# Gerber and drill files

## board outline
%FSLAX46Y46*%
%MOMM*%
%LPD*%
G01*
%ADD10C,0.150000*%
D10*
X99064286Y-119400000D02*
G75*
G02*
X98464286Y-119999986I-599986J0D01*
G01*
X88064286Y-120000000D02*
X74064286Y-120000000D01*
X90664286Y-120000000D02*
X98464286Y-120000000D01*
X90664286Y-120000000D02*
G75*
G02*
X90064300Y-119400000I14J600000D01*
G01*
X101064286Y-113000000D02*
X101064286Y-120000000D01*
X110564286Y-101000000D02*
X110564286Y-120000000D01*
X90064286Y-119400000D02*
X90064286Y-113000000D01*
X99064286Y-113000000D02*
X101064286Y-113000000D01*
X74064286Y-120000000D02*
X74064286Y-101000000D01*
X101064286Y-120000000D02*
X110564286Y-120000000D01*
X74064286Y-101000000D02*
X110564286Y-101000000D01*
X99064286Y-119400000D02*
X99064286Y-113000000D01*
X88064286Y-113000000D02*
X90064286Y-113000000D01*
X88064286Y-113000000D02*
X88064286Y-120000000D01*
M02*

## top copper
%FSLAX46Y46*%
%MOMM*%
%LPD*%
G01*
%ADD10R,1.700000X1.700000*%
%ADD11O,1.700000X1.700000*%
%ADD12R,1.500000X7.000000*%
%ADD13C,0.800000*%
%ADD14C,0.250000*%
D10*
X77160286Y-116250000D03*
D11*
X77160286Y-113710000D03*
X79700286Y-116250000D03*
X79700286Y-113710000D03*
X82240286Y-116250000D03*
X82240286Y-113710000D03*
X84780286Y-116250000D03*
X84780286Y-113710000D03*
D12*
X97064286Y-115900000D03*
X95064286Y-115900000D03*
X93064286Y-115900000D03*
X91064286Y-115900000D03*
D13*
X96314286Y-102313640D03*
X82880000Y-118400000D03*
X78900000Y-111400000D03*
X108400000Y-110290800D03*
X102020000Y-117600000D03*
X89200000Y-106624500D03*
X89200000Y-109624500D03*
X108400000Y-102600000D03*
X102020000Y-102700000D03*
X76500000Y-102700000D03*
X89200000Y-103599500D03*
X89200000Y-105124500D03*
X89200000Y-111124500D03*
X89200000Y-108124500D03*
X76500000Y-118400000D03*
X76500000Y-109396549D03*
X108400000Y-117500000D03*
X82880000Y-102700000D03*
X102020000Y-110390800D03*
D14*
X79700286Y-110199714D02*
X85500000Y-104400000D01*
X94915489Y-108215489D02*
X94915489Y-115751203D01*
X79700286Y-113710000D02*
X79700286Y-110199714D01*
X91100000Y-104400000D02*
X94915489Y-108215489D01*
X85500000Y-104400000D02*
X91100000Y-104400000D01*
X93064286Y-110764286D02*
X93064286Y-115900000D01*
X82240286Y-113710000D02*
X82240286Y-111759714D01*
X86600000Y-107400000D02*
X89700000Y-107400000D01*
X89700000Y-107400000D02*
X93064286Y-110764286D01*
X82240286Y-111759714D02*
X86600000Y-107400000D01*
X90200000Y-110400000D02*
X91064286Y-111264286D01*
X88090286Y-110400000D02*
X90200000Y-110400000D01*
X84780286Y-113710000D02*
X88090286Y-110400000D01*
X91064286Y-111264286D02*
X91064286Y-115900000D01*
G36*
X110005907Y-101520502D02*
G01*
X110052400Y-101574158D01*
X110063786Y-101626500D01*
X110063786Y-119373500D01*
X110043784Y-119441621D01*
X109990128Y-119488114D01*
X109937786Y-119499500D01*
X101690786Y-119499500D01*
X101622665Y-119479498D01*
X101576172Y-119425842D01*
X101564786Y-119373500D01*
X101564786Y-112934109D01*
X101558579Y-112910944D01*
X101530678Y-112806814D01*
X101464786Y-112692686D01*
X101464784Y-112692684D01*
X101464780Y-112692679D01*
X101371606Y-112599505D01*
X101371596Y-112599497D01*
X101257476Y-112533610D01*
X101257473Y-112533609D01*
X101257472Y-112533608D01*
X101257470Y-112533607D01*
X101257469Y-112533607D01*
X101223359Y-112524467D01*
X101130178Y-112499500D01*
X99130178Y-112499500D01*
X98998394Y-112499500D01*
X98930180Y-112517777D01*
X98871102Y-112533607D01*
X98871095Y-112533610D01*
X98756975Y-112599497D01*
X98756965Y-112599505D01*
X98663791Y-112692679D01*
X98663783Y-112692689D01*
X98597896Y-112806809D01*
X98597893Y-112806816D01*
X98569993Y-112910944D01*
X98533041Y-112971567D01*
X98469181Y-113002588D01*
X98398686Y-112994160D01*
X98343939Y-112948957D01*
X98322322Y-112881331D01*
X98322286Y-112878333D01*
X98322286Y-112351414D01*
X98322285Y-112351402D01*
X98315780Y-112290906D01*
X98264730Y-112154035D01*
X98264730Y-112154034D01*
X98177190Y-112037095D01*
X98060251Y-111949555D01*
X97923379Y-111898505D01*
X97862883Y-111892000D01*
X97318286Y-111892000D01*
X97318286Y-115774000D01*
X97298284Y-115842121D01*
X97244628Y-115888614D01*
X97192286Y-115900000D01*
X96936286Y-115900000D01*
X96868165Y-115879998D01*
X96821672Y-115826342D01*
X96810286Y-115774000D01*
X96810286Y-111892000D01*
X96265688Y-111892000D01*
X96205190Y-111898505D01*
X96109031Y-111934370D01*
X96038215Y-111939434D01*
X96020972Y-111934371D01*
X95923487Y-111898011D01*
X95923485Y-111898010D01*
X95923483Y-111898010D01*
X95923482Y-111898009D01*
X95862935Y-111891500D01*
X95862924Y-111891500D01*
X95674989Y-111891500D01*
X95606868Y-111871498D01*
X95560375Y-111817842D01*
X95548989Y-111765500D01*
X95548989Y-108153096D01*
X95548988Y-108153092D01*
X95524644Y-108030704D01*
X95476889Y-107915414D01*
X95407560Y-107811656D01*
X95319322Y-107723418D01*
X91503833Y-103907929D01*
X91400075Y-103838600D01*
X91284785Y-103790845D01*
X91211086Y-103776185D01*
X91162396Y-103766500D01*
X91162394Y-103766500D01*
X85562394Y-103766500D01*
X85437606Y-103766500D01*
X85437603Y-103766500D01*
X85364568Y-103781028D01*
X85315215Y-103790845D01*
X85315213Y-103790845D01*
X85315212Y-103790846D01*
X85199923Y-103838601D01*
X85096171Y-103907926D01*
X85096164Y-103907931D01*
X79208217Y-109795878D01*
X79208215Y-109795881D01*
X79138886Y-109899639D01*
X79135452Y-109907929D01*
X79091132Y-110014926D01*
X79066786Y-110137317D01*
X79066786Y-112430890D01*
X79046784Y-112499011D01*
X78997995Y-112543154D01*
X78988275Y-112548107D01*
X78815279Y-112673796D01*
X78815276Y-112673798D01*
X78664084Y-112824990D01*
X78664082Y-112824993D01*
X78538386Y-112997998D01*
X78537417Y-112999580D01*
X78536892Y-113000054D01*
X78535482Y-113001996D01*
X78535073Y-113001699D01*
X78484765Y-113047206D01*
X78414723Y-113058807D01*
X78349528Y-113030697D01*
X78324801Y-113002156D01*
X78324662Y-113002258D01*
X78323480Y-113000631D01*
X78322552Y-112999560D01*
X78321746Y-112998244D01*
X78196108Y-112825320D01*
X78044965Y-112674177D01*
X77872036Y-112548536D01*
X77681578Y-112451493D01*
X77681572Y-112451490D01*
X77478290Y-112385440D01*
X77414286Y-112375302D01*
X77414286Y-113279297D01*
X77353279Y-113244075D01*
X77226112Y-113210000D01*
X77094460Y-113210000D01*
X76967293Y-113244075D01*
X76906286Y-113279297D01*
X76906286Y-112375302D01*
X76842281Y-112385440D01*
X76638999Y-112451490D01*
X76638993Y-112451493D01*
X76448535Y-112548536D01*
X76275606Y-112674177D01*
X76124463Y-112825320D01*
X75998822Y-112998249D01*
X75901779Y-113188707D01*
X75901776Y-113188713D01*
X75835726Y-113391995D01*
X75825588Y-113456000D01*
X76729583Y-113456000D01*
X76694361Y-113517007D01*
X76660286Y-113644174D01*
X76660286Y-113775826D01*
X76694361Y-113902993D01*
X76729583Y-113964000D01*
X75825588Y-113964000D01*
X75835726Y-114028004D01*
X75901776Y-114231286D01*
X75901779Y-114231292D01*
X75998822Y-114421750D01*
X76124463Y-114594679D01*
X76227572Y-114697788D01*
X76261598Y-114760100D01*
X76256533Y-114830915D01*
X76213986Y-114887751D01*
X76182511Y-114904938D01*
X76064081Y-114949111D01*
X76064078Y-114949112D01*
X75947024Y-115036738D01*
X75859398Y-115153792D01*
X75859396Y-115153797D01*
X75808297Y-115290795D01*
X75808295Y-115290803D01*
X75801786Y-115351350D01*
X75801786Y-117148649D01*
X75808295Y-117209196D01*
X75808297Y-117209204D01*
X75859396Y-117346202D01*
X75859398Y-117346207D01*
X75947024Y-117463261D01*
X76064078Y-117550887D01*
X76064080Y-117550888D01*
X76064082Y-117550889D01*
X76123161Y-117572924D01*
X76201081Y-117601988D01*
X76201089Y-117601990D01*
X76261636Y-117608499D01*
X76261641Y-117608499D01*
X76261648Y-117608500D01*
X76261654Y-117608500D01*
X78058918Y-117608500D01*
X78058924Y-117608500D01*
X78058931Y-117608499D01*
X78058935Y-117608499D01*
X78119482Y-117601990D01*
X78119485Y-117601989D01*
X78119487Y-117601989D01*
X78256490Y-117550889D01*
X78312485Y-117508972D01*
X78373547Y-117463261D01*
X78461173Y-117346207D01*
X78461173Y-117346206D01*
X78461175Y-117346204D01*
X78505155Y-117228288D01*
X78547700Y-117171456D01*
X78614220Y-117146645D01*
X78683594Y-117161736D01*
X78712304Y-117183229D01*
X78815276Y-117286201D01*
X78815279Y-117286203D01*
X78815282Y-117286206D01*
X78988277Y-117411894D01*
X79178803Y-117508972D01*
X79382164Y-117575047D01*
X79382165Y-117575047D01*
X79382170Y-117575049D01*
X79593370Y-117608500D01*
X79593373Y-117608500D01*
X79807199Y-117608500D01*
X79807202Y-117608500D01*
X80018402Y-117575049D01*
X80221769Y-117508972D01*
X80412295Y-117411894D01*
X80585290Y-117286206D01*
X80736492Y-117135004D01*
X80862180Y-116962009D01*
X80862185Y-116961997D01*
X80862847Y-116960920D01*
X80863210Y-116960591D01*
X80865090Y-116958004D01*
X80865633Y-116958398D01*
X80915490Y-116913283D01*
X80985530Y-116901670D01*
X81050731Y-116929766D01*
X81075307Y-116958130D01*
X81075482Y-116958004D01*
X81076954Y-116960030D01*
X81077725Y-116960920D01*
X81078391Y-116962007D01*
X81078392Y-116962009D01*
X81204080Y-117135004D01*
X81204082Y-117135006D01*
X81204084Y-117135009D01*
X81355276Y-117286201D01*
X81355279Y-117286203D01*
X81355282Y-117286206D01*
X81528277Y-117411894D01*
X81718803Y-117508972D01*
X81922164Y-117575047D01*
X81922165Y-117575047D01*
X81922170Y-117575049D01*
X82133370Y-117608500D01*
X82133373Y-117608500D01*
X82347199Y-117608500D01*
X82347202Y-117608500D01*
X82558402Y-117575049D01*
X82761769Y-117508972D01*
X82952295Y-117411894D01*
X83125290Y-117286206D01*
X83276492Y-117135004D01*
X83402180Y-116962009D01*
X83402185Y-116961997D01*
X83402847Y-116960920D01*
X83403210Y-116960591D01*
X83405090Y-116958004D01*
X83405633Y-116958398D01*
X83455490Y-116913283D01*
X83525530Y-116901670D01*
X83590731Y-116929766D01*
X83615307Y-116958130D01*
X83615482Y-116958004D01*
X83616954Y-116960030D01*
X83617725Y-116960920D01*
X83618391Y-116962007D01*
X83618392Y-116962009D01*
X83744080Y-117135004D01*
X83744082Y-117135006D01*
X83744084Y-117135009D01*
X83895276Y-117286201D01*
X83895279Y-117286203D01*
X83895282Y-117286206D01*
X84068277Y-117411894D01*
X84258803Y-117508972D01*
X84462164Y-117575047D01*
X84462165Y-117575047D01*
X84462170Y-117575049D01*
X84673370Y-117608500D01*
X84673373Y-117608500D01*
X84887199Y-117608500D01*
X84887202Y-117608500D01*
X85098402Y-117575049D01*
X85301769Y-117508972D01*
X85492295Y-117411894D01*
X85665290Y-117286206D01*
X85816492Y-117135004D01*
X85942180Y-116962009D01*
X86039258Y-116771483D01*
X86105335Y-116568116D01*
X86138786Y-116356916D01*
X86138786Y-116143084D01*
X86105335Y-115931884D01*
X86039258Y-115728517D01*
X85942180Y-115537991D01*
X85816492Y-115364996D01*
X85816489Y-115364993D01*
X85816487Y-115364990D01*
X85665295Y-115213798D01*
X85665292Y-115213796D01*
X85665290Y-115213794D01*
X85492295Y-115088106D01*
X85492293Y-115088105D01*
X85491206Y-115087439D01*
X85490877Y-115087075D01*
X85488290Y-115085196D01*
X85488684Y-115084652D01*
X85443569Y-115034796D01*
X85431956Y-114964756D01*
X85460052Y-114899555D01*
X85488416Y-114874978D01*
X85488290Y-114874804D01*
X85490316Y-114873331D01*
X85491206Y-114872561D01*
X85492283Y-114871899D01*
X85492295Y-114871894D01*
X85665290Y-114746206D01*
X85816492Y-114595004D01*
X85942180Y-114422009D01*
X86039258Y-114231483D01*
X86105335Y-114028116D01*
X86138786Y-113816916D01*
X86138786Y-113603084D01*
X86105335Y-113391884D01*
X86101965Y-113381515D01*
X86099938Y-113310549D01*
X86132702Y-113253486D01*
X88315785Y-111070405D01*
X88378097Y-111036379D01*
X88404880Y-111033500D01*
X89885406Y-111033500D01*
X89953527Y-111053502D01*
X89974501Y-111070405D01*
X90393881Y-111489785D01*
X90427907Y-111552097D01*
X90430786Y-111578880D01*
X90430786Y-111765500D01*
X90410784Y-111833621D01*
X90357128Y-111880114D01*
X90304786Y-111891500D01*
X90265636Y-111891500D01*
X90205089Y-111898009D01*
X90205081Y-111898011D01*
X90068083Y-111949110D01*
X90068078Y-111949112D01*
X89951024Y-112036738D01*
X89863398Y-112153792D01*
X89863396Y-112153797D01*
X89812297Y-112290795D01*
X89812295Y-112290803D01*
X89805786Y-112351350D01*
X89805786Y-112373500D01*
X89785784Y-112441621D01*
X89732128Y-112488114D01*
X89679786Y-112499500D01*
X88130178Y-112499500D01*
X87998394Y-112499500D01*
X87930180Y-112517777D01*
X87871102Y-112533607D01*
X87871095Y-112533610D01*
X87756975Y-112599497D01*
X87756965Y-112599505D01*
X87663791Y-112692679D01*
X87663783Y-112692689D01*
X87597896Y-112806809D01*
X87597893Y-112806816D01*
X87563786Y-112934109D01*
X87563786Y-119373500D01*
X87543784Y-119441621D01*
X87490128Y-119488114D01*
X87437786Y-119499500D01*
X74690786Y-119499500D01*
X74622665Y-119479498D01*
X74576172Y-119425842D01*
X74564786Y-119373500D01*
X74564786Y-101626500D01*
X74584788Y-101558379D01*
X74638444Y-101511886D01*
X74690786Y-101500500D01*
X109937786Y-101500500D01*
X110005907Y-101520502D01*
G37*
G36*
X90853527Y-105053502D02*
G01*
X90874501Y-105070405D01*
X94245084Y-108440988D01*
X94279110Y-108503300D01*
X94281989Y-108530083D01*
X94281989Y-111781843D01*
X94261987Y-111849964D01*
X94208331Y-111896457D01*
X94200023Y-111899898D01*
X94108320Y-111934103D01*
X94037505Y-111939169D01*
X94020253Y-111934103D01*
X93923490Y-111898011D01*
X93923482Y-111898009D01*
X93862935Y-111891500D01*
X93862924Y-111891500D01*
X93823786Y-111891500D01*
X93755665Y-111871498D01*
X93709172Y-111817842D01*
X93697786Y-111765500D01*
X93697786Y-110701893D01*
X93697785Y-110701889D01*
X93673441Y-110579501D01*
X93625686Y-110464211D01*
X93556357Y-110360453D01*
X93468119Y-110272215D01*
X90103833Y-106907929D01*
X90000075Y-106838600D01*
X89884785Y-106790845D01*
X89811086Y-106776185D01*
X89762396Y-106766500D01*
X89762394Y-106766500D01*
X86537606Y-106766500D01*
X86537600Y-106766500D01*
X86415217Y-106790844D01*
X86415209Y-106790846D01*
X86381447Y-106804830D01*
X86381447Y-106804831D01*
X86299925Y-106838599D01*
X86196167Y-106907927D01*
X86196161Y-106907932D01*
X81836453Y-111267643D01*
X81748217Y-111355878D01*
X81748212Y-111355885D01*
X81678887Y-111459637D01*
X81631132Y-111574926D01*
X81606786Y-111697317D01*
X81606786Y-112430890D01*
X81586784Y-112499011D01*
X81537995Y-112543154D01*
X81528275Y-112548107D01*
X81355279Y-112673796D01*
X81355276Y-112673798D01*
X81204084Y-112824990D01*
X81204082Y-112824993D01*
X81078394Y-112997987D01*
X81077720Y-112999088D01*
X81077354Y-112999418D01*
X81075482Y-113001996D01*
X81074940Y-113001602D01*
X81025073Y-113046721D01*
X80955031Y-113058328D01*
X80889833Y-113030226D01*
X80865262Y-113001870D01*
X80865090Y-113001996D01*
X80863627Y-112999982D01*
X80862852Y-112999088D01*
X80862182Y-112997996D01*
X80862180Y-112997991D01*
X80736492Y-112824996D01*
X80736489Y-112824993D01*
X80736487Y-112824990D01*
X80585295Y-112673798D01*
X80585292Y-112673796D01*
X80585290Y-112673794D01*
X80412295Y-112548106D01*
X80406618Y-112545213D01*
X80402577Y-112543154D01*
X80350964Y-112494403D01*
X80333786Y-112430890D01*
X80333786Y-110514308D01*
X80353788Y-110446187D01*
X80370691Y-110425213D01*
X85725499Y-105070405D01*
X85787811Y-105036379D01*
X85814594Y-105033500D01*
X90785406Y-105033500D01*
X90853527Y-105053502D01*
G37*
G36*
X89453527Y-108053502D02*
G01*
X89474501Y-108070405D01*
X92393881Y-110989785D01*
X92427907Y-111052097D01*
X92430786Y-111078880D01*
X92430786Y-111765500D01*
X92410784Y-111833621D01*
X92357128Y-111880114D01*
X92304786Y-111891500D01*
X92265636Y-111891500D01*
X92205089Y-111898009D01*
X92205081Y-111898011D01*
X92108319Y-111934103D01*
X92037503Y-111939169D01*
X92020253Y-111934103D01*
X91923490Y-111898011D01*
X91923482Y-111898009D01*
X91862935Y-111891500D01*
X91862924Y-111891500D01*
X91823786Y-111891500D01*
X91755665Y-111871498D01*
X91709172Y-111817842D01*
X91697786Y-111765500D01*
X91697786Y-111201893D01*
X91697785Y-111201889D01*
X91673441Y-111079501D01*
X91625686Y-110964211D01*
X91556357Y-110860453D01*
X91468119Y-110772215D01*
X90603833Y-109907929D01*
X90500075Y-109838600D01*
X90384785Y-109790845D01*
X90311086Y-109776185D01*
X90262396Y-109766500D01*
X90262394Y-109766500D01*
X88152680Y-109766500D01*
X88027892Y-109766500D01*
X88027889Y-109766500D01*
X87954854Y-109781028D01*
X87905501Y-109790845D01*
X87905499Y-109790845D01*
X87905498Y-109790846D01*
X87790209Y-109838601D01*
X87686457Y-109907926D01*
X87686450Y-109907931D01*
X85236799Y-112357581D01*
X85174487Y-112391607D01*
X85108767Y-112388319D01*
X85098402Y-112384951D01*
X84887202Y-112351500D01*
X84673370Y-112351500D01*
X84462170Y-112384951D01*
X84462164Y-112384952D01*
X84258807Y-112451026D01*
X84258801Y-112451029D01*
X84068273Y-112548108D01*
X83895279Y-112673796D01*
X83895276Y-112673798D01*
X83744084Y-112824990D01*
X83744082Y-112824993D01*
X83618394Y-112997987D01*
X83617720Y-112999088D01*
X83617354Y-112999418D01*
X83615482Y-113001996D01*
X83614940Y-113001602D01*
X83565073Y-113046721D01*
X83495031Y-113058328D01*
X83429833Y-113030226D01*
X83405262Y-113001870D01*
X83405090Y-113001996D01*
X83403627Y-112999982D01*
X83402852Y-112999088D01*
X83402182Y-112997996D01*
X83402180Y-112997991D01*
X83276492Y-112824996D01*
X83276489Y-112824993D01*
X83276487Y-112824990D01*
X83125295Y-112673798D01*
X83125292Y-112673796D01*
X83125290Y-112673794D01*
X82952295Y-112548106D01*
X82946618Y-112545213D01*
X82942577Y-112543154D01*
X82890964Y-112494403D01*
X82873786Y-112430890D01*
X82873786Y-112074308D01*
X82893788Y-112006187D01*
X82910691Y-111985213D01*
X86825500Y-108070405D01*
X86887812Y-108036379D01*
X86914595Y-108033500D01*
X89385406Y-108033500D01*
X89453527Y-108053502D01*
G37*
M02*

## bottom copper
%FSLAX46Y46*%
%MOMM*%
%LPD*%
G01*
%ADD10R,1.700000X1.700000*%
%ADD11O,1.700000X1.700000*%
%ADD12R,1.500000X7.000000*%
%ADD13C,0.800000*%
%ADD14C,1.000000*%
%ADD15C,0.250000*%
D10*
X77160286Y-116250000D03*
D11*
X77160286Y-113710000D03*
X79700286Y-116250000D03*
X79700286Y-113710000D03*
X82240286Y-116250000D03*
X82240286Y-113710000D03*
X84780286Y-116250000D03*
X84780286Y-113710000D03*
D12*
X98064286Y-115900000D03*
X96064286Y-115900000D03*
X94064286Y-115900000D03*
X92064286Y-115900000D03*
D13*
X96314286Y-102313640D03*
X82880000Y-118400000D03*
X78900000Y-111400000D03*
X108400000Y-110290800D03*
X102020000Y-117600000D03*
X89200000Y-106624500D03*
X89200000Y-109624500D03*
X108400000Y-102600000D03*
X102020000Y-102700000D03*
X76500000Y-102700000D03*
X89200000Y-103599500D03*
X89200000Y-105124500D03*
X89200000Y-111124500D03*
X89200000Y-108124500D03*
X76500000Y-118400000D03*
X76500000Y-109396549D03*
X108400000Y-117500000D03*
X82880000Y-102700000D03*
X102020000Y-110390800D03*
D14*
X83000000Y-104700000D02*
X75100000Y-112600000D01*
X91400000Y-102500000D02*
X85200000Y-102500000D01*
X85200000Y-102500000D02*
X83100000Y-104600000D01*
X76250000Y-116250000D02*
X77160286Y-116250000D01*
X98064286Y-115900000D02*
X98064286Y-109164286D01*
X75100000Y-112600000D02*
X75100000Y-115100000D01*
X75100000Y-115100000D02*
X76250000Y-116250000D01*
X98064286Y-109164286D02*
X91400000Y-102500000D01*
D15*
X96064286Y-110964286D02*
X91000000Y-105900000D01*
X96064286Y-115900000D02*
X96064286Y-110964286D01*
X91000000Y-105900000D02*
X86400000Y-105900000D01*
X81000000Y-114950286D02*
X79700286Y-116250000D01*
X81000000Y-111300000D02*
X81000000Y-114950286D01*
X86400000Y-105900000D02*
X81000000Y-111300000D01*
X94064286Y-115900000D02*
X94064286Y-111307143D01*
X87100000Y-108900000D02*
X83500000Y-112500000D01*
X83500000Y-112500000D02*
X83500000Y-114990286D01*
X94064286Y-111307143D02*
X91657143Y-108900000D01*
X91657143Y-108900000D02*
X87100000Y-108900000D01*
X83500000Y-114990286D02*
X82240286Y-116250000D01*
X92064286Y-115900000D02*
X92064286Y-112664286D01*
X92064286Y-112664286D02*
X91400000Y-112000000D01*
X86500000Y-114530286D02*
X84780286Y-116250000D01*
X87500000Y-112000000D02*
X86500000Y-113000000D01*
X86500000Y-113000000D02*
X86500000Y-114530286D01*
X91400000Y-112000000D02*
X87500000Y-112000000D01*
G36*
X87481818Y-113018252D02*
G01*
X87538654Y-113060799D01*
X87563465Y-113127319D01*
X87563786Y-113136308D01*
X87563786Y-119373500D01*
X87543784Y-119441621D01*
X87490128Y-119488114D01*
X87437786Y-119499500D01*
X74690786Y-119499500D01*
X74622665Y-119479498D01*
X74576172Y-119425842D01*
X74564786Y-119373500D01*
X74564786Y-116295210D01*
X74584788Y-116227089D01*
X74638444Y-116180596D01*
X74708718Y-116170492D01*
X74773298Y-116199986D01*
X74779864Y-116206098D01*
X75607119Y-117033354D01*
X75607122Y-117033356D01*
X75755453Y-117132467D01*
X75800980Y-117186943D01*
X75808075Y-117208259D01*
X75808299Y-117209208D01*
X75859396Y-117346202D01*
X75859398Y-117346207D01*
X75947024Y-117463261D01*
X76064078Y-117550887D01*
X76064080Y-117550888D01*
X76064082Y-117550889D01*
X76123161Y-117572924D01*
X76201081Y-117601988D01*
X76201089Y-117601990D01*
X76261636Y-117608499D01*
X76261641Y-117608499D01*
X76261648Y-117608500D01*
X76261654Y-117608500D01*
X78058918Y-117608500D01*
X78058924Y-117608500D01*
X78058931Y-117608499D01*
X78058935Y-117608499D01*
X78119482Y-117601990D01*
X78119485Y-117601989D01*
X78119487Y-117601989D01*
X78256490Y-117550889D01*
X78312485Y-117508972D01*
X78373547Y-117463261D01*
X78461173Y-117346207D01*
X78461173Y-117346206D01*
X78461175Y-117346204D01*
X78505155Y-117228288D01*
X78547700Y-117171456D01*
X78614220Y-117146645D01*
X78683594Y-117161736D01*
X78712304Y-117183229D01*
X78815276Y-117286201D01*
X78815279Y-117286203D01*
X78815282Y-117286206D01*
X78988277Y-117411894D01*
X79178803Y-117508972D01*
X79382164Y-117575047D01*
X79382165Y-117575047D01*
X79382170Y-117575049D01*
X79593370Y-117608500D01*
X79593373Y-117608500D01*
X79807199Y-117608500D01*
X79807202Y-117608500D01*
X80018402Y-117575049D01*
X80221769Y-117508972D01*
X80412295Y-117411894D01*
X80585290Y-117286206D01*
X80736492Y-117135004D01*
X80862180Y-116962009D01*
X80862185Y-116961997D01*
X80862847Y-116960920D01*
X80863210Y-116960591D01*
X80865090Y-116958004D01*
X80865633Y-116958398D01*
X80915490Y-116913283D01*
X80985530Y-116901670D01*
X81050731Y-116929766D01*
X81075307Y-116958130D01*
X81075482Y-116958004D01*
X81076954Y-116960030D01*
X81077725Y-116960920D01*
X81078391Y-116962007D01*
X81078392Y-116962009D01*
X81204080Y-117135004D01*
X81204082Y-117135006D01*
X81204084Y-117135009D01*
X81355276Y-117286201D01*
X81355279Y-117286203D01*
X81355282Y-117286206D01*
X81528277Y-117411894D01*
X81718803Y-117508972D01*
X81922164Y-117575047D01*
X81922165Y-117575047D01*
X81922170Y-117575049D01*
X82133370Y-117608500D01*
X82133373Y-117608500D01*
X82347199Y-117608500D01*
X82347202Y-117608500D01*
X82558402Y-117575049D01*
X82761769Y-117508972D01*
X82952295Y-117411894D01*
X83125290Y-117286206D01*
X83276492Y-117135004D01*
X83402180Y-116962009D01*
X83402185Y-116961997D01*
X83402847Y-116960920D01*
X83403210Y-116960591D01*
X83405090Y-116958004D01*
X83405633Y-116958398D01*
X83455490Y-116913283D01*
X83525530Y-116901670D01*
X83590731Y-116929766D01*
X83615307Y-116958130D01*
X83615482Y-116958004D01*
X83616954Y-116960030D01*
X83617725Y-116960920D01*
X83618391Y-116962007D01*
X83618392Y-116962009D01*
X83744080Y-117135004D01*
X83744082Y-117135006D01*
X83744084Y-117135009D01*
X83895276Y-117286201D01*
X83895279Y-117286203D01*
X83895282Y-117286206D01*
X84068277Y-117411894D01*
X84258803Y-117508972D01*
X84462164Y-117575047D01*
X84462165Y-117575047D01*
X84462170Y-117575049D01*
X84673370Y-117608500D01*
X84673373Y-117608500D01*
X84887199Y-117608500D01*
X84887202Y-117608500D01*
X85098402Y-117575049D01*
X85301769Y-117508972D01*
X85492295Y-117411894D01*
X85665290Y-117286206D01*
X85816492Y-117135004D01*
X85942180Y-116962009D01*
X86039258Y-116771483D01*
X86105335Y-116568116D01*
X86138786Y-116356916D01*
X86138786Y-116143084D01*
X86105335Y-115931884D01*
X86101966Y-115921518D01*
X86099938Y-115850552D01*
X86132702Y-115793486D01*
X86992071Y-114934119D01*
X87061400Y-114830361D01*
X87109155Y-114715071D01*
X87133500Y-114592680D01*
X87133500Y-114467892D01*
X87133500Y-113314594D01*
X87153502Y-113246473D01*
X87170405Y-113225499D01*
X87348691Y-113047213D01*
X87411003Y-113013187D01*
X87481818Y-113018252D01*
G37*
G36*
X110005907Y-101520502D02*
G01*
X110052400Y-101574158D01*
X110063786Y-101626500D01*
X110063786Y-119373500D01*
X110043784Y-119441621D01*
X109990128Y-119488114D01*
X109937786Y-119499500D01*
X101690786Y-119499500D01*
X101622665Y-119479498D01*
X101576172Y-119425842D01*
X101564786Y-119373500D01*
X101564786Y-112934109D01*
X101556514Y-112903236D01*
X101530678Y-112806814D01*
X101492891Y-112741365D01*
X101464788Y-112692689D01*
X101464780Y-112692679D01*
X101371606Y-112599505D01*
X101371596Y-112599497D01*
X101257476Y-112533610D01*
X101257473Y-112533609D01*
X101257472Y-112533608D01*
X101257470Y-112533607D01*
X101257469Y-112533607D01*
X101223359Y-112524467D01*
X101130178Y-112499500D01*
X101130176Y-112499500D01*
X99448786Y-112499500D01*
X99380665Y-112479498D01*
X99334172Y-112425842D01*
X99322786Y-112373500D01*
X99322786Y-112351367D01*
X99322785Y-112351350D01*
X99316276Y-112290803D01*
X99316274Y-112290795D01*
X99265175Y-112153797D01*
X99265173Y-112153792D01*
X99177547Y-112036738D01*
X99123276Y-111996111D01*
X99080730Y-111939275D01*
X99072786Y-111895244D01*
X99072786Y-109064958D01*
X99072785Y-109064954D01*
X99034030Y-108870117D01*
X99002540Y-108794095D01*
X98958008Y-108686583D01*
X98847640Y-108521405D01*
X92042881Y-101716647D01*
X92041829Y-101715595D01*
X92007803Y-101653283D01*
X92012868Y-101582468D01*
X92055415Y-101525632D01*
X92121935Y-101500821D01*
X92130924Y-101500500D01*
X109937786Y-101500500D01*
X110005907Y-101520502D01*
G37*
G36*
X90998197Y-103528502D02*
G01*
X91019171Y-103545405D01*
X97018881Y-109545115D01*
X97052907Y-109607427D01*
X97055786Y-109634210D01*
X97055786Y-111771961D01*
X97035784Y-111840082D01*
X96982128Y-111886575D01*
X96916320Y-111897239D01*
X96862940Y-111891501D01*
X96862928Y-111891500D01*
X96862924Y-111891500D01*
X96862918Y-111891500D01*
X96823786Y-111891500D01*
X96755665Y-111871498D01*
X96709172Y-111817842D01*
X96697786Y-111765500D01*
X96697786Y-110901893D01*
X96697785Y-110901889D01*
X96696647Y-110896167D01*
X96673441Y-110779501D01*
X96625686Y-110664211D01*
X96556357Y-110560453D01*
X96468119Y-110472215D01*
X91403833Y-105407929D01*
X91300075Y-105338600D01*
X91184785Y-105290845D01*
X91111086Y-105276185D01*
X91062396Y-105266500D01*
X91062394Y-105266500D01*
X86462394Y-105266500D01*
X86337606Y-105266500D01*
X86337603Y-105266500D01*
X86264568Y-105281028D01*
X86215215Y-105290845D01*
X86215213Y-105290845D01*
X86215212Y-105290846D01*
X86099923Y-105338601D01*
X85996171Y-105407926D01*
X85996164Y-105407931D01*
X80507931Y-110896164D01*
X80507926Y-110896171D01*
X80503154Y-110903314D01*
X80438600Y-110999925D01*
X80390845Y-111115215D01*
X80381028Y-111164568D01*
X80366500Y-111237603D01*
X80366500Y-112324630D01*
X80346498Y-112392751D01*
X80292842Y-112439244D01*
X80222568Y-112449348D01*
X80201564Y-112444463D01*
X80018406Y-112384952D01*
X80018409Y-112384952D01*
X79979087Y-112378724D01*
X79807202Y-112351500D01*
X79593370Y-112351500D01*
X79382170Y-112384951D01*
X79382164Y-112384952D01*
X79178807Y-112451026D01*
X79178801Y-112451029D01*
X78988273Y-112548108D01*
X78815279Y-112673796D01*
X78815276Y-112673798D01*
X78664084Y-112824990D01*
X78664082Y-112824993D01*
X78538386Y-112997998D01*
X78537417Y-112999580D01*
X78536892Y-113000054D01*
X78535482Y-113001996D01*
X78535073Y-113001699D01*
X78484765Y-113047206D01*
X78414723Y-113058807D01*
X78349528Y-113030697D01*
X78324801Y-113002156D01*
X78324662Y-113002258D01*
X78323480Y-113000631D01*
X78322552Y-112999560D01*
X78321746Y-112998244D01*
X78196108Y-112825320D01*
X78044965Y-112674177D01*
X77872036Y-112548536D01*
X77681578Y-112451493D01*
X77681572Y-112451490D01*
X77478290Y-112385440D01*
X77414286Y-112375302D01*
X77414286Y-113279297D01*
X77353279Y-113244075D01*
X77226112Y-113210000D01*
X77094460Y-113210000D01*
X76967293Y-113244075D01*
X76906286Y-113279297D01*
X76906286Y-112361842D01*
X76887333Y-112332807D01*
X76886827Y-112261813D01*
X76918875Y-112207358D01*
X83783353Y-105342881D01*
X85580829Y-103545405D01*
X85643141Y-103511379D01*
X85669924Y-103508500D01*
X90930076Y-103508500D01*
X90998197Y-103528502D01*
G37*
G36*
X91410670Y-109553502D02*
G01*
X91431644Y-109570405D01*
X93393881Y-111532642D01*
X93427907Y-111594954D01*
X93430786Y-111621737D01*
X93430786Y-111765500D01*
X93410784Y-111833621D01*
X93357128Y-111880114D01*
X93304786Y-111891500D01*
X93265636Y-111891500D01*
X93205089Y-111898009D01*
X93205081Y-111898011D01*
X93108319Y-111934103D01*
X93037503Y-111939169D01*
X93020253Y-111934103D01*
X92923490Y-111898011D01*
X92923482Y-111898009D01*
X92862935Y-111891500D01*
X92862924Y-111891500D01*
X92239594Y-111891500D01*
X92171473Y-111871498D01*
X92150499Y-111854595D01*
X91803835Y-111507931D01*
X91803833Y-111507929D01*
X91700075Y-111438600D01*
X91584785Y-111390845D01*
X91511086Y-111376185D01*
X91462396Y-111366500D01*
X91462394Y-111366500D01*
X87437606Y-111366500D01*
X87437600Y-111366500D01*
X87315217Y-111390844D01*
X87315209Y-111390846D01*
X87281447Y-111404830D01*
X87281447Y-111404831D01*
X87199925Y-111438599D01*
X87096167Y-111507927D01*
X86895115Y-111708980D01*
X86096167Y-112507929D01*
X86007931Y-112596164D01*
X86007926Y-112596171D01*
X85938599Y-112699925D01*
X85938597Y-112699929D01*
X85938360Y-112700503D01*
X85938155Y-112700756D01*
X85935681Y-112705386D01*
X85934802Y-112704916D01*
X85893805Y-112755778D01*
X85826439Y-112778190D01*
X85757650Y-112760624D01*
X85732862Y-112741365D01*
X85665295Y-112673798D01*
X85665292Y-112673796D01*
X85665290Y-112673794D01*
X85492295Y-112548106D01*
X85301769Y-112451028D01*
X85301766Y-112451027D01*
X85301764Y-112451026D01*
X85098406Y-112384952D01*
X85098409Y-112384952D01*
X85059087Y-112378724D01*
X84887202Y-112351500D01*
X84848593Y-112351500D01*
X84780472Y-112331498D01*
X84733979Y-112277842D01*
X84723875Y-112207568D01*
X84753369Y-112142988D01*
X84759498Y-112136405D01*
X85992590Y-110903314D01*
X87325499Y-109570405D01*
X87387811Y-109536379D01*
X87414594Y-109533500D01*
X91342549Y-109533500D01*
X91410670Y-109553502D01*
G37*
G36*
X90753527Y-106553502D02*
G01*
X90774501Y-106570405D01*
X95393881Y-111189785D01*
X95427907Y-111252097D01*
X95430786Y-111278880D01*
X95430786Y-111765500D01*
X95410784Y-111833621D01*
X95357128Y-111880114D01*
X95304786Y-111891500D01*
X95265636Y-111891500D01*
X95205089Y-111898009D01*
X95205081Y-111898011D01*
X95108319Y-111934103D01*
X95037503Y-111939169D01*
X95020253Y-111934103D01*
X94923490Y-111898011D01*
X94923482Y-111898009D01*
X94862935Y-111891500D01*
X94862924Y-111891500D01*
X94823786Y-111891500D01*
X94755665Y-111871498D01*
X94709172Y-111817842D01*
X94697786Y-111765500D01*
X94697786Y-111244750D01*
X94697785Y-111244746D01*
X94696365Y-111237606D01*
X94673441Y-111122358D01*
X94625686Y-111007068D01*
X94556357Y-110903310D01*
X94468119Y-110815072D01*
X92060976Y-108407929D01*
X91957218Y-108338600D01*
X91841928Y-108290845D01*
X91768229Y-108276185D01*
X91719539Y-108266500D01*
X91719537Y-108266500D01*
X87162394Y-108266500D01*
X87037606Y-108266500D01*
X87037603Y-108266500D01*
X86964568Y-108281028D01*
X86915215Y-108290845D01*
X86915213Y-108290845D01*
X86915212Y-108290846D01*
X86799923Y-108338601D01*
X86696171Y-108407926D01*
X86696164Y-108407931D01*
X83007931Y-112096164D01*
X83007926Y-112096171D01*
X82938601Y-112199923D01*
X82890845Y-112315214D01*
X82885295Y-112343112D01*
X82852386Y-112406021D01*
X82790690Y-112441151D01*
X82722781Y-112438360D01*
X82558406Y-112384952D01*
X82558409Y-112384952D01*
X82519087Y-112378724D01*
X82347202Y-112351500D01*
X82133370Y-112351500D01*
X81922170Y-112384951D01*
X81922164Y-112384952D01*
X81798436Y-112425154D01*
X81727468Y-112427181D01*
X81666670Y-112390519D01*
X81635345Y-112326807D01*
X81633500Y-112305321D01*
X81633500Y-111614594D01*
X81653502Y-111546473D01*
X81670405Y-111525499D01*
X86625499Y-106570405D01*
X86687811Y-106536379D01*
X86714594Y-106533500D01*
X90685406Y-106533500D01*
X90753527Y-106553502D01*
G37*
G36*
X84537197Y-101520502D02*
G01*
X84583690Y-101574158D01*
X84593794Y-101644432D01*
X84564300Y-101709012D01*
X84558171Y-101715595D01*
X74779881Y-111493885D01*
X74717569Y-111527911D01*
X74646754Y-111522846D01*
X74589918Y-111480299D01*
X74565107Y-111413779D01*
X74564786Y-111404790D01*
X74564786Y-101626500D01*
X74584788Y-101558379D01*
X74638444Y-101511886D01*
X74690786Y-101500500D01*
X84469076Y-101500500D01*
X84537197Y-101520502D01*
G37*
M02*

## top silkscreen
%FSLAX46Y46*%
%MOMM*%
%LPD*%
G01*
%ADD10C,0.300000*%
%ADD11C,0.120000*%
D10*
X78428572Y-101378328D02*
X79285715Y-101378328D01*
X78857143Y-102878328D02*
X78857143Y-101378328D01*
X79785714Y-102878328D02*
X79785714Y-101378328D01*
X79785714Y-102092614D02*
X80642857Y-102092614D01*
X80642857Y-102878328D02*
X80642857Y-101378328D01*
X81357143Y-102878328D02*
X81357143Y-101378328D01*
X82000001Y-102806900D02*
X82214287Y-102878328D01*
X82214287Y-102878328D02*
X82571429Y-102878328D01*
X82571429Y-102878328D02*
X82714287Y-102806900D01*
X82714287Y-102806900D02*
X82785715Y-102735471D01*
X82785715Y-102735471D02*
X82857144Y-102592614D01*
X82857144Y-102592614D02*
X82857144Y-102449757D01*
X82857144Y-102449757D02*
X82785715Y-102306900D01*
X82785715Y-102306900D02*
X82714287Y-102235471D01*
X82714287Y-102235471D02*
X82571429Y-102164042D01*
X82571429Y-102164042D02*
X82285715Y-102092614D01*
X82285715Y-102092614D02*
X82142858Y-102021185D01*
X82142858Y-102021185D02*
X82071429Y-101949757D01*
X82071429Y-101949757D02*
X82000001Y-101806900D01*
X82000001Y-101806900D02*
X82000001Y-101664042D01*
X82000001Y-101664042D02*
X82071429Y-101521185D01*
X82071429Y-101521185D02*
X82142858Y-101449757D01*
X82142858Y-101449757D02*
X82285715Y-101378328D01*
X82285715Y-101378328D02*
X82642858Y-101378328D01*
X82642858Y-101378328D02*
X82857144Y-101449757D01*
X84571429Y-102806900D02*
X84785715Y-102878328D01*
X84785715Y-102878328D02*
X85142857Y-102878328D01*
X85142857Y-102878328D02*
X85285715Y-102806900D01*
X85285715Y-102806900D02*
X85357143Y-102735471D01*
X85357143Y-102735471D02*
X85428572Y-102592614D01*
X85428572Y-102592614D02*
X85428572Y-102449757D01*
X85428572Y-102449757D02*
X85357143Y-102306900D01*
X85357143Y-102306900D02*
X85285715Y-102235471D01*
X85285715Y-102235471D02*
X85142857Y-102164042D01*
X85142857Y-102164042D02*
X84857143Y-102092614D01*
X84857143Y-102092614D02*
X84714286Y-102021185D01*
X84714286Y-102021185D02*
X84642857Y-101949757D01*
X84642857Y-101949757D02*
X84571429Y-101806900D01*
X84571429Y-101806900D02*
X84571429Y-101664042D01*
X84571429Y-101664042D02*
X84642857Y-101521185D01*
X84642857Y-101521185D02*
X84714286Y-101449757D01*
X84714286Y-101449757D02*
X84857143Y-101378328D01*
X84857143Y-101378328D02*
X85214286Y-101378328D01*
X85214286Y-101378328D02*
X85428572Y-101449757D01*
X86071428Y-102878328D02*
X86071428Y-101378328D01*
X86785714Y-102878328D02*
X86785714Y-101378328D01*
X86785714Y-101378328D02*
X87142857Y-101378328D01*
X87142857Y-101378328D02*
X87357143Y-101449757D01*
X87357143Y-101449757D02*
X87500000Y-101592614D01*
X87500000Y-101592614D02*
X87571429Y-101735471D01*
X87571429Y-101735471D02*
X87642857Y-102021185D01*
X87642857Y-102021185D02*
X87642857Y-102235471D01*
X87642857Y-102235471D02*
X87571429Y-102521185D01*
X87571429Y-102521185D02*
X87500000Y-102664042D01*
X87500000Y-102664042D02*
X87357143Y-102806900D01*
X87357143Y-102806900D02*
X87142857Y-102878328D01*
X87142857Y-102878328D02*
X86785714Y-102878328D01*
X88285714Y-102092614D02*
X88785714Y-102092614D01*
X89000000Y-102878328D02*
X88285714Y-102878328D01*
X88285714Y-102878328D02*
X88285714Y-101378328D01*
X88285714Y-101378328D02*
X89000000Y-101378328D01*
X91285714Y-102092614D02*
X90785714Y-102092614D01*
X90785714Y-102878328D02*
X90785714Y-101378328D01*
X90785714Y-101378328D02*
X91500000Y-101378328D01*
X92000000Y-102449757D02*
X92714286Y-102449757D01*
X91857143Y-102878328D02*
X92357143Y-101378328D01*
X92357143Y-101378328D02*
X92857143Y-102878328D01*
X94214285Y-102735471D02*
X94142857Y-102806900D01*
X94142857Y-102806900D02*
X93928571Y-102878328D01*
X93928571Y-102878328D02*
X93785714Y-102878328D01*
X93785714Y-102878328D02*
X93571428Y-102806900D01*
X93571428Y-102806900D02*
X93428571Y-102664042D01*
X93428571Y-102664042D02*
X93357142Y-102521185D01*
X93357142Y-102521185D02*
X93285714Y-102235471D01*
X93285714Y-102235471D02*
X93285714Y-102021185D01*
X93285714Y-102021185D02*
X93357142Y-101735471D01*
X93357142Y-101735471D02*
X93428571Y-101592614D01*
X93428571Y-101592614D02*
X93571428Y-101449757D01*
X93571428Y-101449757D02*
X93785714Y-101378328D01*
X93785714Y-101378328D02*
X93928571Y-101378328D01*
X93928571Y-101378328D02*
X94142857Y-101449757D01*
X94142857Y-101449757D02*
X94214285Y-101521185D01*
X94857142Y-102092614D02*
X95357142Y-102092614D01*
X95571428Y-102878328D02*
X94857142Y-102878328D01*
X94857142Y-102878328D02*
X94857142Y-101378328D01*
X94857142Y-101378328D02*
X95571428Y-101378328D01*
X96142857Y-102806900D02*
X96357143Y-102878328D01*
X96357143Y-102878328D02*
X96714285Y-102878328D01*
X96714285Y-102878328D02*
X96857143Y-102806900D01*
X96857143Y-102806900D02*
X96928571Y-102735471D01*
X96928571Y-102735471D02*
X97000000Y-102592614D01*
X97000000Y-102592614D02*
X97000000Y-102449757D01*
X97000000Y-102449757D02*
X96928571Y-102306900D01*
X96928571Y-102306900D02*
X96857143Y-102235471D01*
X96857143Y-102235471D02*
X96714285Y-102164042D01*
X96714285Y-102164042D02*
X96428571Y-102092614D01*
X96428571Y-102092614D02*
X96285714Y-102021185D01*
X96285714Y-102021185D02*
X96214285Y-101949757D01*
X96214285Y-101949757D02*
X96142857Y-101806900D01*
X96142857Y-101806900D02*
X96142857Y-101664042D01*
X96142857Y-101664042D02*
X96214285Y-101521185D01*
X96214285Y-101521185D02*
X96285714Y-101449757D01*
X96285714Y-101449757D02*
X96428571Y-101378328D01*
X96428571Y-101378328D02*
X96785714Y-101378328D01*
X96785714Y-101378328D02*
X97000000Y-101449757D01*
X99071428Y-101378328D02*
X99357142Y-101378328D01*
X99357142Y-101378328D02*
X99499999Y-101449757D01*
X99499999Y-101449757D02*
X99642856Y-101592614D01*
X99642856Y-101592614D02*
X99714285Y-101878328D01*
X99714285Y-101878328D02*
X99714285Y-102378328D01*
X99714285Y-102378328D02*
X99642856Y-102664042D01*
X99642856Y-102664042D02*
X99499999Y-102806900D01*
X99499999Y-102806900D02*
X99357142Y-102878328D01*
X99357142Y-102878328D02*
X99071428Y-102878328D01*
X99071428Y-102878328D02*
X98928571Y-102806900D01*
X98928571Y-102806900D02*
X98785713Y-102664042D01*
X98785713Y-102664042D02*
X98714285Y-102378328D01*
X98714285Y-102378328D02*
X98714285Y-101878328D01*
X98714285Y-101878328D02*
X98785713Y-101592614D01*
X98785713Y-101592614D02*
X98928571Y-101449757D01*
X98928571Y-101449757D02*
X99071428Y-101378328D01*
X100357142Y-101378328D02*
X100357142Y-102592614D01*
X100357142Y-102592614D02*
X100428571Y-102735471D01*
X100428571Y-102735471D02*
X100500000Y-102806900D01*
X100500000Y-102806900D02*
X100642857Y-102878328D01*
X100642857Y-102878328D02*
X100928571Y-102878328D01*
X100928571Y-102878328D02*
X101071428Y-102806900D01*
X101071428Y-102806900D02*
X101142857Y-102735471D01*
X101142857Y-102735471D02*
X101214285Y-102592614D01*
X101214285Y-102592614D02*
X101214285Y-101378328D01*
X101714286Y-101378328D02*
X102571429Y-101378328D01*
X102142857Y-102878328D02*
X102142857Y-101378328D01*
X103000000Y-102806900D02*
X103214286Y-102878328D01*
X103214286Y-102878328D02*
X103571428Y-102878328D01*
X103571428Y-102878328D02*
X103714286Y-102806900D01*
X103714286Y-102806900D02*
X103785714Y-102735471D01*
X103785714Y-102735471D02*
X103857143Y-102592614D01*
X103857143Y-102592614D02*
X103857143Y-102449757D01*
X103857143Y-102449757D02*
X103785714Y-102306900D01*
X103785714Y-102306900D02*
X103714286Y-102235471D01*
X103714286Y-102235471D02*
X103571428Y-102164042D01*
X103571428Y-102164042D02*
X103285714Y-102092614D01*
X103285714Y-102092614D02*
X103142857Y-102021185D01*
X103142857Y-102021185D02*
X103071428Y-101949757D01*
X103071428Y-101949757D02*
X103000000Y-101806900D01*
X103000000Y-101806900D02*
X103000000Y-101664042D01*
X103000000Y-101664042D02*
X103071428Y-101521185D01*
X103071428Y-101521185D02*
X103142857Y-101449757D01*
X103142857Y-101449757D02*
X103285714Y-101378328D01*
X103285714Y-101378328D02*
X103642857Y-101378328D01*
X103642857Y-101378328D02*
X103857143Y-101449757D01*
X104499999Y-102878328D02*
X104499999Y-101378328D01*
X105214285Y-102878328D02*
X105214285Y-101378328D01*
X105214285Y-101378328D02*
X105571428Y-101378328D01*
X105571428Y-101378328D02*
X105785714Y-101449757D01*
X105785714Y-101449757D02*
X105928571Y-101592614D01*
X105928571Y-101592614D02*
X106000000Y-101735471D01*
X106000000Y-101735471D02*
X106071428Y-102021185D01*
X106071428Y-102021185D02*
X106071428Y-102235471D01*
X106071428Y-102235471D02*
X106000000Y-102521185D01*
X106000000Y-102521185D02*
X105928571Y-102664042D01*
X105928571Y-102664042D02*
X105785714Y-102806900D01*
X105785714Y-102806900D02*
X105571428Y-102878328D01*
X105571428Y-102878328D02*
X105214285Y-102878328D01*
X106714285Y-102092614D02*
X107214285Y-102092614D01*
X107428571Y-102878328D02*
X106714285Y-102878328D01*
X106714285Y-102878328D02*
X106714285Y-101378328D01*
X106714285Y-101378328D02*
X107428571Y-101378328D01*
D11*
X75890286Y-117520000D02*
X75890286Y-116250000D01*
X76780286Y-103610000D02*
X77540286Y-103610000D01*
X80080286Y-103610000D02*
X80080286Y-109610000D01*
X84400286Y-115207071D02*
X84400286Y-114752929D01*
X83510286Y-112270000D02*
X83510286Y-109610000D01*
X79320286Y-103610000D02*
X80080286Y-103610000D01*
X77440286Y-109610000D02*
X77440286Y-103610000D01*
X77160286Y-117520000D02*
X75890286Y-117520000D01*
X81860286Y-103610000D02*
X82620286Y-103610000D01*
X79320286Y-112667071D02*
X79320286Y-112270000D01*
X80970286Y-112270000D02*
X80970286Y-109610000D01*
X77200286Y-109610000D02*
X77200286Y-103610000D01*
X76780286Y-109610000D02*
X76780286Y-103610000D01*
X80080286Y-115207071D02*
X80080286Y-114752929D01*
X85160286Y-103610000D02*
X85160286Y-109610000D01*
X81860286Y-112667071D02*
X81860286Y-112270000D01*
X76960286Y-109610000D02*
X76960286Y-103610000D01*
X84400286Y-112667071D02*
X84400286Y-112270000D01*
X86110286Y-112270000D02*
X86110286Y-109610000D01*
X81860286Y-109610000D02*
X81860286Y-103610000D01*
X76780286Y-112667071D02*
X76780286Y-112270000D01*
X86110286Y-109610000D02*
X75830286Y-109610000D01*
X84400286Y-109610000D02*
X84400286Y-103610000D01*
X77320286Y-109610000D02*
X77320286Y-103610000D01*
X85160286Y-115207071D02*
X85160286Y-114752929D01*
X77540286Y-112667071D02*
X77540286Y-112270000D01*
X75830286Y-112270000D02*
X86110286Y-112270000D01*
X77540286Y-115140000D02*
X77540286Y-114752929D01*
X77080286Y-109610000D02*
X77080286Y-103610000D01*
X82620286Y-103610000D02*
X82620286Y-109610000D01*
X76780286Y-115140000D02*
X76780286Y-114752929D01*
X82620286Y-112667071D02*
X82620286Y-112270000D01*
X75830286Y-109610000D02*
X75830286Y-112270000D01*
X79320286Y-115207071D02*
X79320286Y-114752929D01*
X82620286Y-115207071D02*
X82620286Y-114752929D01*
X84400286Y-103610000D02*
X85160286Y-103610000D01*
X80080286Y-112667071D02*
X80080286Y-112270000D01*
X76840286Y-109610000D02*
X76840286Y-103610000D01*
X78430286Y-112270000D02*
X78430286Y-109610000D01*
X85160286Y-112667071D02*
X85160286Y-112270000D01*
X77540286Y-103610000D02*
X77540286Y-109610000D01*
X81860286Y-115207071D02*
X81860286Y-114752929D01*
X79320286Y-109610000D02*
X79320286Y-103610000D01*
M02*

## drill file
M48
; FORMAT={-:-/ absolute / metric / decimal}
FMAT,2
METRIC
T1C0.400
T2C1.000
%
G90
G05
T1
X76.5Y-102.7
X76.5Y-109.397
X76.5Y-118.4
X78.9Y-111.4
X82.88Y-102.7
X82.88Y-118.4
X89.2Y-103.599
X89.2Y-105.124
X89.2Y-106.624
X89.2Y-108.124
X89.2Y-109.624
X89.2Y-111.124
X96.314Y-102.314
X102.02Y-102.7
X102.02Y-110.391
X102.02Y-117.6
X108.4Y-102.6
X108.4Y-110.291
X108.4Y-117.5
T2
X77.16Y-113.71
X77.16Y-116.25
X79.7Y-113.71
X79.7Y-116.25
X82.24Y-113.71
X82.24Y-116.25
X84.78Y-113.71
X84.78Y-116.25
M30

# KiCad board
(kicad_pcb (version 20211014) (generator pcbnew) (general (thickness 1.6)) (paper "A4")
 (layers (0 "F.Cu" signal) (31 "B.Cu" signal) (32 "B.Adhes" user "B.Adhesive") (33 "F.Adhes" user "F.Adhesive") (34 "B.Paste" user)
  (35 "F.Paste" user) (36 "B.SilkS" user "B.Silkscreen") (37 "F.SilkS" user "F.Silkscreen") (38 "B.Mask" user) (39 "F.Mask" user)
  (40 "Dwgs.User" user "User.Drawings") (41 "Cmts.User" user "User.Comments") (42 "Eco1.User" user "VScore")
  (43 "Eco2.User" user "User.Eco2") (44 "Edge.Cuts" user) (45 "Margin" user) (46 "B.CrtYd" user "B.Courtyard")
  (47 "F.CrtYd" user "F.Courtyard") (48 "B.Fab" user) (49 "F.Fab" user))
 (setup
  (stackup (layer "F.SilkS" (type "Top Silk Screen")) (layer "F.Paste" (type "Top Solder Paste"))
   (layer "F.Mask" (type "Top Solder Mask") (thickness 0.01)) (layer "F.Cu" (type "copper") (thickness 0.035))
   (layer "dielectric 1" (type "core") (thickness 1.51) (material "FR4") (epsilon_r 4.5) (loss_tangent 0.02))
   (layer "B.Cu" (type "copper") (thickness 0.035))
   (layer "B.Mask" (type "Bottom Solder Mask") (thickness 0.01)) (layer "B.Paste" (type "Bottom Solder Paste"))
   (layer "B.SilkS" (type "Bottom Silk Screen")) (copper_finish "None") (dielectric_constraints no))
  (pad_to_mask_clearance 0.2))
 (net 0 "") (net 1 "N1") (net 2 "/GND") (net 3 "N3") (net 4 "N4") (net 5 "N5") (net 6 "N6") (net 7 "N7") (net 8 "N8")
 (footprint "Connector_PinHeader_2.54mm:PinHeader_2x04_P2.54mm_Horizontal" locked (layer "F.Cu") (at 77.160286 116.25 90)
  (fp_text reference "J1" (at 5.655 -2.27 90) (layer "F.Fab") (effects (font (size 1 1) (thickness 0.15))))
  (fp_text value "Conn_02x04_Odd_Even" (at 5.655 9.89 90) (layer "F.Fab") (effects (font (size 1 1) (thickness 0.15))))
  (fp_line (start -1.27 -1.27) (end 0 -1.27) (layer "F.SilkS") (width 0.12))
  (fp_line (start 12.64 -0.38) (end 12.64 0.38) (layer "F.SilkS") (width 0.12))
  (fp_line (start 12.64 2.92) (end 6.64 2.92) (layer "F.SilkS") (width 0.12))
  (fp_line (start 1.042929 7.24) (end 1.497071 7.24) (layer "F.SilkS") (width 0.12))
  (fp_line (start 3.98 6.35) (end 6.64 6.35) (layer "F.SilkS") (width 0.12))
  (fp_line (start 12.64 2.16) (end 12.64 2.92) (layer "F.SilkS") (width 0.12))
  (fp_line (start 6.64 0.28) (end 12.64 0.28) (layer "F.SilkS") (width 0.12))
  (fp_line (start -1.27 0) (end -1.27 -1.27) (layer "F.SilkS") (width 0.12))
  (fp_line (start 12.64 4.7) (end 12.64 5.46) (layer "F.SilkS") (width 0.12))
  (fp_line (start 3.582929 2.16) (end 3.98 2.16) (layer "F.SilkS") (width 0.12))
  (fp_line (start 3.98 3.81) (end 6.64 3.81) (layer "F.SilkS") (width 0.12))
  (fp_line (start 6.64 0.04) (end 12.64 0.04) (layer "F.SilkS") (width 0.12))
  (fp_line (start 6.64 -0.38) (end 12.64 -0.38) (layer "F.SilkS") (width 0.12))
  (fp_line (start 1.042929 2.92) (end 1.497071 2.92) (layer "F.SilkS") (width 0.12))
  (fp_line (start 12.64 8) (end 6.64 8) (layer "F.SilkS") (width 0.12))
  (fp_line (start 3.582929 4.7) (end 3.98 4.7) (layer "F.SilkS") (width 0.12))
  (fp_line (start 6.64 -0.2) (end 12.64 -0.2) (layer "F.SilkS") (width 0.12))
  (fp_line (start 3.582929 7.24) (end 3.98 7.24) (layer "F.SilkS") (width 0.12))
  (fp_line (start 3.98 8.95) (end 6.64 8.95) (layer "F.SilkS") (width 0.12))
  (fp_line (start 6.64 4.7) (end 12.64 4.7) (layer "F.SilkS") (width 0.12))
  (fp_line (start 3.582929 -0.38) (end 3.98 -0.38) (layer "F.SilkS") (width 0.12))
  (fp_line (start 6.64 8.95) (end 6.64 -1.33) (layer "F.SilkS") (width 0.12))
  (fp_line (start 6.64 7.24) (end 12.64 7.24) (layer "F.SilkS") (width 0.12))
  (fp_line (start 6.64 0.16) (end 12.64 0.16) (layer "F.SilkS") (width 0.12))
  (fp_line (start 1.042929 8) (end 1.497071 8) (layer "F.SilkS") (width 0.12))
  (fp_line (start 3.582929 0.38) (end 3.98 0.38) (layer "F.SilkS") (width 0.12))
  (fp_line (start 3.98 -1.33) (end 3.98 8.95) (layer "F.SilkS") (width 0.12))
  (fp_line (start 1.11 0.38) (end 1.497071 0.38) (layer "F.SilkS") (width 0.12))
  (fp_line (start 6.64 -0.08) (end 12.64 -0.08) (layer "F.SilkS") (width 0.12))
  (fp_line (start 12.64 5.46) (end 6.64 5.46) (layer "F.SilkS") (width 0.12))
  (fp_line (start 1.11 -0.38) (end 1.497071 -0.38) (layer "F.SilkS") (width 0.12))
  (fp_line (start 3.582929 5.46) (end 3.98 5.46) (layer "F.SilkS") (width 0.12))
  (fp_line (start 6.64 -1.33) (end 3.98 -1.33) (layer "F.SilkS") (width 0.12))
  (fp_line (start 1.042929 2.16) (end 1.497071 2.16) (layer "F.SilkS") (width 0.12))
  (fp_line (start 1.042929 5.46) (end 1.497071 5.46) (layer "F.SilkS") (width 0.12))
  (fp_line (start 12.64 7.24) (end 12.64 8) (layer "F.SilkS") (width 0.12))
  (fp_line (start 3.582929 2.92) (end 3.98 2.92) (layer "F.SilkS") (width 0.12))
  (fp_line (start 6.64 -0.32) (end 12.64 -0.32) (layer "F.SilkS") (width 0.12))
  (fp_line (start 3.98 1.27) (end 6.64 1.27) (layer "F.SilkS") (width 0.12))
  (fp_line (start 3.582929 8) (end 3.98 8) (layer "F.SilkS") (width 0.12))
  (fp_line (start 12.64 0.38) (end 6.64 0.38) (layer "F.SilkS") (width 0.12))
  (fp_line (start 1.042929 4.7) (end 1.497071 4.7) (layer "F.SilkS") (width 0.12))
  (fp_line (start 6.64 2.16) (end 12.64 2.16) (layer "F.SilkS") (width 0.12))
  (pad "1" thru_hole rect locked (at 0 0 90) (size 1.7 1.7) (drill 1) (layers *.Cu *.Mask) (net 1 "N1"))
  (pad "2" thru_hole oval locked (at 2.54 0 90) (size 1.7 1.7) (drill 1) (layers *.Cu *.Mask) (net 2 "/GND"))
  (pad "3" thru_hole oval locked (at 0 2.54 90) (size 1.7 1.7) (drill 1) (layers *.Cu *.Mask) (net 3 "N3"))
  (pad "4" thru_hole oval locked (at 2.54 2.54 90) (size 1.7 1.7) (drill 1) (layers *.Cu *.Mask) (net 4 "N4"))
  (pad "5" thru_hole oval locked (at 0 5.08 90) (size 1.7 1.7) (drill 1) (layers *.Cu *.Mask) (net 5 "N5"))
  (pad "6" thru_hole oval locked (at 2.54 5.08 90) (size 1.7 1.7) (drill 1) (layers *.Cu *.Mask) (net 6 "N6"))
  (pad "7" thru_hole oval locked (at 0 7.62 90) (size 1.7 1.7) (drill 1) (layers *.Cu *.Mask) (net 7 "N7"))
  (pad "8" thru_hole oval locked (at 2.54 7.62 90) (size 1.7 1.7) (drill 1) (layers *.Cu *.Mask) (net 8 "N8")))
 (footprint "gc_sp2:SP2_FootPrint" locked (layer "B.Cu") (at 98.064286 115.9 180)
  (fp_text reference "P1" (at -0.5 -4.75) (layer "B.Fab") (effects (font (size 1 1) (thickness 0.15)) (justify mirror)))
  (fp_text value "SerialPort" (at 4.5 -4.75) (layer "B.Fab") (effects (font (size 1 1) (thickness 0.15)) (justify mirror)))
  (pad "1" smd rect locked (at 0 0 180) (size 1.5 7) (layers "B.Cu" "B.Paste" "B.Mask") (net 1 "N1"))
  (pad "2" smd rect locked (at 1 0 180) (size 1.5 7) (layers "F.Cu" "F.Paste" "F.Mask") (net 2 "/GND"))
  (pad "3" smd rect locked (at 2 0 180) (size 1.5 7) (layers "B.Cu" "B.Paste" "B.Mask") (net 3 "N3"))
  (pad "4" smd rect locked (at 3 0 180) (size 1.5 7) (layers "F.Cu" "F.Paste" "F.Mask") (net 4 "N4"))
  (pad "5" smd rect locked (at 4 0 180) (size 1.5 7) (layers "B.Cu" "B.Paste" "B.Mask") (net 5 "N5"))
  (pad "6" smd rect locked (at 5 0 180) (size 1.5 7) (layers "F.Cu" "F.Paste" "F.Mask") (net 6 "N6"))
  (pad "7" smd rect locked (at 6 0 180) (size 1.5 7) (layers "B.Cu" "B.Paste" "B.Mask") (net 7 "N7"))
  (pad "8" smd rect locked (at 7 0 180) (size 1.5 7) (layers "F.Cu" "F.Paste" "F.Mask") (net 8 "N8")))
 (gr_arc (start 99.064286 119.4) (mid 98.88855 119.824264) (end 98.464286 120) (layer "Edge.Cuts") (width 0.15))
 (gr_line (start 88.064286 120) (end 74.064286 120) (layer "Edge.Cuts") (width 0.15))
 (gr_line (start 90.664286 120) (end 98.464286 120) (layer "Edge.Cuts") (width 0.15))
 (gr_arc (start 90.664286 120) (mid 90.240022 119.824264) (end 90.064286 119.4) (layer "Edge.Cuts") (width 0.15))
 (gr_line (start 101.064286 113) (end 101.064286 120) (layer "Edge.Cuts") (width 0.15))
 (gr_line (start 110.564286 101) (end 110.564286 120) (layer "Edge.Cuts") (width 0.15))
 (gr_line (start 90.064286 119.4) (end 90.064286 113) (layer "Edge.Cuts") (width 0.15))
 (gr_line (start 99.064286 113) (end 101.064286 113) (layer "Edge.Cuts") (width 0.15))
 (gr_line (start 74.064286 120) (end 74.064286 101) (layer "Edge.Cuts") (width 0.15))
 (gr_line (start 101.064286 120) (end 110.564286 120) (layer "Edge.Cuts") (width 0.15))
 (gr_line (start 74.064286 101) (end 110.564286 101) (layer "Edge.Cuts") (width 0.15))
 (gr_line (start 99.064286 119.4) (end 99.064286 113) (layer "Edge.Cuts") (width 0.15))
 (gr_line (start 88.064286 113) (end 90.064286 113) (layer "Edge.Cuts") (width 0.15))
 (gr_line (start 88.064286 113) (end 88.064286 120) (layer "Edge.Cuts") (width 0.15))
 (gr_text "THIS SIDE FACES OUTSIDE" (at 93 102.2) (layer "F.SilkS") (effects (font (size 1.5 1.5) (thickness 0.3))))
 (segment (start 83 104.7) (end 75.1 112.6) (width 1) (layer "B.Cu") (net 1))
 (segment (start 91.4 102.5) (end 85.2 102.5) (width 1) (layer "B.Cu") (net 1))
 (segment (start 85.2 102.5) (end 83.1 104.6) (width 1) (layer "B.Cu") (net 1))
 (segment (start 76.25 116.25) (end 77.160286 116.25) (width 1) (layer "B.Cu") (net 1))
 (segment (start 98.064286 115.9) (end 98.064286 109.164286) (width 1) (layer "B.Cu") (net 1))
 (segment (start 75.1 112.6) (end 75.1 115.1) (width 1) (layer "B.Cu") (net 1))
 (segment (start 75.1 115.1) (end 76.25 116.25) (width 1) (layer "B.Cu") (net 1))
 (segment (start 98.064286 109.164286) (end 91.4 102.5) (width 1) (layer "B.Cu") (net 1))
 (segment (start 96.064286 110.964286) (end 91 105.9) (width 0.25) (layer "B.Cu") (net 3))
 (segment (start 96.064286 115.9) (end 96.064286 110.964286) (width 0.25) (layer "B.Cu") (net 3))
 (segment (start 91 105.9) (end 86.4 105.9) (width 0.25) (layer "B.Cu") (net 3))
 (segment (start 81 114.950286) (end 79.700286 116.25) (width 0.25) (layer "B.Cu") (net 3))
 (segment (start 81 111.3) (end 81 114.950286) (width 0.25) (layer "B.Cu") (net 3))
 (segment (start 86.4 105.9) (end 81 111.3) (width 0.25) (layer "B.Cu") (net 3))
 (segment (start 79.700286 110.199714) (end 85.5 104.4) (width 0.25) (layer "F.Cu") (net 4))
 (segment (start 94.915489 108.215489) (end 94.915489 115.751203) (width 0.25) (layer "F.Cu") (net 4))
 (segment (start 79.700286 113.71) (end 79.700286 110.199714) (width 0.25) (layer "F.Cu") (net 4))
 (segment (start 91.1 104.4) (end 94.915489 108.215489) (width 0.25) (layer "F.Cu") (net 4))
 (segment (start 85.5 104.4) (end 91.1 104.4) (width 0.25) (layer "F.Cu") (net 4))
 (segment (start 94.064286 115.9) (end 94.064286 111.307143) (width 0.25) (layer "B.Cu") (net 5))
 (segment (start 87.1 108.9) (end 83.5 112.5) (width 0.25) (layer "B.Cu") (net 5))
 (segment (start 83.5 112.5) (end 83.5 114.990286) (width 0.25) (layer "B.Cu") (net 5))
 (segment (start 94.064286 111.307143) (end 91.657143 108.9) (width 0.25) (layer "B.Cu") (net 5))
 (segment (start 91.657143 108.9) (end 87.1 108.9) (width 0.25) (layer "B.Cu") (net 5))
 (segment (start 83.5 114.990286) (end 82.240286 116.25) (width 0.25) (layer "B.Cu") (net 5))
 (segment (start 93.064286 110.764286) (end 93.064286 115.9) (width 0.25) (layer "F.Cu") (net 6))
 (segment (start 82.240286 113.71) (end 82.240286 111.759714) (width 0.25) (layer "F.Cu") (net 6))
 (segment (start 86.6 107.4) (end 89.7 107.4) (width 0.25) (layer "F.Cu") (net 6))
 (segment (start 89.7 107.4) (end 93.064286 110.764286) (width 0.25) (layer "F.Cu") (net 6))
 (segment (start 82.240286 111.759714) (end 86.6 107.4) (width 0.25) (layer "F.Cu") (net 6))
 (segment (start 92.064286 115.9) (end 92.064286 112.664286) (width 0.25) (layer "B.Cu") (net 7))
 (segment (start 92.064286 112.664286) (end 91.4 112) (width 0.25) (layer "B.Cu") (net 7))
 (segment (start 86.5 114.530286) (end 84.780286 116.25) (width 0.25) (layer "B.Cu") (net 7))
 (segment (start 87.5 112) (end 86.5 113) (width 0.25) (layer "B.Cu") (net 7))
 (segment (start 86.5 113) (end 86.5 114.530286) (width 0.25) (layer "B.Cu") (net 7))
 (segment (start 91.4 112) (end 87.5 112) (width 0.25) (layer "B.Cu") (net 7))
 (segment (start 90.2 110.4) (end 91.064286 111.264286) (width 0.25) (layer "F.Cu") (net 8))
 (segment (start 88.090286 110.4) (end 90.2 110.4) (width 0.25) (layer "F.Cu") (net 8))
 (segment (start 84.780286 113.71) (end 88.090286 110.4) (width 0.25) (layer "F.Cu") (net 8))
 (segment (start 91.064286 111.264286) (end 91.064286 115.9) (width 0.25) (layer "F.Cu") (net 8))
 (via (at 96.314286 102.31364) (size 0.8) (drill 0.4) (layers "F.Cu" "B.Cu") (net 2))
 (via (at 82.88 118.4) (size 0.8) (drill 0.4) (layers "F.Cu" "B.Cu") (free) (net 2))
 (via (at 78.9 111.4) (size 0.8) (drill 0.4) (layers "F.Cu" "B.Cu") (free) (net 2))
 (via (at 108.4 110.2908) (size 0.8) (drill 0.4) (layers "F.Cu" "B.Cu") (free) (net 2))
 (via (at 102.02 117.6) (size 0.8) (drill 0.4) (layers "F.Cu" "B.Cu") (free) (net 2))
 (via (at 89.2 106.6245) (size 0.8) (drill 0.4) (layers "F.Cu" "B.Cu") (free) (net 2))
 (via (at 89.2 109.6245) (size 0.8) (drill 0.4) (layers "F.Cu" "B.Cu") (free) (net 2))
 (via (at 108.4 102.6) (size 0.8) (drill 0.4) (layers "F.Cu" "B.Cu") (free) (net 2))
 (via (at 102.02 102.7) (size 0.8) (drill 0.4) (layers "F.Cu" "B.Cu") (free) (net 2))
 (via (at 76.5 102.7) (size 0.8) (drill 0.4) (layers "F.Cu" "B.Cu") (free) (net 2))
 (via (at 89.2 103.5995) (size 0.8) (drill 0.4) (layers "F.Cu" "B.Cu") (free) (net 2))
 (via (at 89.2 105.1245) (size 0.8) (drill 0.4) (layers "F.Cu" "B.Cu") (free) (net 2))
 (via (at 89.2 111.1245) (size 0.8) (drill 0.4) (layers "F.Cu" "B.Cu") (free) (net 2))
 (via (at 89.2 108.1245) (size 0.8) (drill 0.4) (layers "F.Cu" "B.Cu") (free) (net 2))
 (via (at 76.5 118.4) (size 0.8) (drill 0.4) (layers "F.Cu" "B.Cu") (free) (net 2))
 (via (at 76.5 109.396549) (size 0.8) (drill 0.4) (layers "F.Cu" "B.Cu") (free) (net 2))
 (via (at 108.4 117.5) (size 0.8) (drill 0.4) (layers "F.Cu" "B.Cu") (free) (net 2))
 (via (at 82.88 102.7) (size 0.8) (drill 0.4) (layers "F.Cu" "B.Cu") (free) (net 2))
 (via (at 102.02 110.3908) (size 0.8) (drill 0.4) (layers "F.Cu" "B.Cu") (free) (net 2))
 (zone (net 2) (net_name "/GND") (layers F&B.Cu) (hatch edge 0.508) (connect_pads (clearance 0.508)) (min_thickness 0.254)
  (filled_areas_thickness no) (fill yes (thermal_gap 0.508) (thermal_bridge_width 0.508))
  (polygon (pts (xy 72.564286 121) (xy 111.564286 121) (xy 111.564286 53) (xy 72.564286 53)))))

